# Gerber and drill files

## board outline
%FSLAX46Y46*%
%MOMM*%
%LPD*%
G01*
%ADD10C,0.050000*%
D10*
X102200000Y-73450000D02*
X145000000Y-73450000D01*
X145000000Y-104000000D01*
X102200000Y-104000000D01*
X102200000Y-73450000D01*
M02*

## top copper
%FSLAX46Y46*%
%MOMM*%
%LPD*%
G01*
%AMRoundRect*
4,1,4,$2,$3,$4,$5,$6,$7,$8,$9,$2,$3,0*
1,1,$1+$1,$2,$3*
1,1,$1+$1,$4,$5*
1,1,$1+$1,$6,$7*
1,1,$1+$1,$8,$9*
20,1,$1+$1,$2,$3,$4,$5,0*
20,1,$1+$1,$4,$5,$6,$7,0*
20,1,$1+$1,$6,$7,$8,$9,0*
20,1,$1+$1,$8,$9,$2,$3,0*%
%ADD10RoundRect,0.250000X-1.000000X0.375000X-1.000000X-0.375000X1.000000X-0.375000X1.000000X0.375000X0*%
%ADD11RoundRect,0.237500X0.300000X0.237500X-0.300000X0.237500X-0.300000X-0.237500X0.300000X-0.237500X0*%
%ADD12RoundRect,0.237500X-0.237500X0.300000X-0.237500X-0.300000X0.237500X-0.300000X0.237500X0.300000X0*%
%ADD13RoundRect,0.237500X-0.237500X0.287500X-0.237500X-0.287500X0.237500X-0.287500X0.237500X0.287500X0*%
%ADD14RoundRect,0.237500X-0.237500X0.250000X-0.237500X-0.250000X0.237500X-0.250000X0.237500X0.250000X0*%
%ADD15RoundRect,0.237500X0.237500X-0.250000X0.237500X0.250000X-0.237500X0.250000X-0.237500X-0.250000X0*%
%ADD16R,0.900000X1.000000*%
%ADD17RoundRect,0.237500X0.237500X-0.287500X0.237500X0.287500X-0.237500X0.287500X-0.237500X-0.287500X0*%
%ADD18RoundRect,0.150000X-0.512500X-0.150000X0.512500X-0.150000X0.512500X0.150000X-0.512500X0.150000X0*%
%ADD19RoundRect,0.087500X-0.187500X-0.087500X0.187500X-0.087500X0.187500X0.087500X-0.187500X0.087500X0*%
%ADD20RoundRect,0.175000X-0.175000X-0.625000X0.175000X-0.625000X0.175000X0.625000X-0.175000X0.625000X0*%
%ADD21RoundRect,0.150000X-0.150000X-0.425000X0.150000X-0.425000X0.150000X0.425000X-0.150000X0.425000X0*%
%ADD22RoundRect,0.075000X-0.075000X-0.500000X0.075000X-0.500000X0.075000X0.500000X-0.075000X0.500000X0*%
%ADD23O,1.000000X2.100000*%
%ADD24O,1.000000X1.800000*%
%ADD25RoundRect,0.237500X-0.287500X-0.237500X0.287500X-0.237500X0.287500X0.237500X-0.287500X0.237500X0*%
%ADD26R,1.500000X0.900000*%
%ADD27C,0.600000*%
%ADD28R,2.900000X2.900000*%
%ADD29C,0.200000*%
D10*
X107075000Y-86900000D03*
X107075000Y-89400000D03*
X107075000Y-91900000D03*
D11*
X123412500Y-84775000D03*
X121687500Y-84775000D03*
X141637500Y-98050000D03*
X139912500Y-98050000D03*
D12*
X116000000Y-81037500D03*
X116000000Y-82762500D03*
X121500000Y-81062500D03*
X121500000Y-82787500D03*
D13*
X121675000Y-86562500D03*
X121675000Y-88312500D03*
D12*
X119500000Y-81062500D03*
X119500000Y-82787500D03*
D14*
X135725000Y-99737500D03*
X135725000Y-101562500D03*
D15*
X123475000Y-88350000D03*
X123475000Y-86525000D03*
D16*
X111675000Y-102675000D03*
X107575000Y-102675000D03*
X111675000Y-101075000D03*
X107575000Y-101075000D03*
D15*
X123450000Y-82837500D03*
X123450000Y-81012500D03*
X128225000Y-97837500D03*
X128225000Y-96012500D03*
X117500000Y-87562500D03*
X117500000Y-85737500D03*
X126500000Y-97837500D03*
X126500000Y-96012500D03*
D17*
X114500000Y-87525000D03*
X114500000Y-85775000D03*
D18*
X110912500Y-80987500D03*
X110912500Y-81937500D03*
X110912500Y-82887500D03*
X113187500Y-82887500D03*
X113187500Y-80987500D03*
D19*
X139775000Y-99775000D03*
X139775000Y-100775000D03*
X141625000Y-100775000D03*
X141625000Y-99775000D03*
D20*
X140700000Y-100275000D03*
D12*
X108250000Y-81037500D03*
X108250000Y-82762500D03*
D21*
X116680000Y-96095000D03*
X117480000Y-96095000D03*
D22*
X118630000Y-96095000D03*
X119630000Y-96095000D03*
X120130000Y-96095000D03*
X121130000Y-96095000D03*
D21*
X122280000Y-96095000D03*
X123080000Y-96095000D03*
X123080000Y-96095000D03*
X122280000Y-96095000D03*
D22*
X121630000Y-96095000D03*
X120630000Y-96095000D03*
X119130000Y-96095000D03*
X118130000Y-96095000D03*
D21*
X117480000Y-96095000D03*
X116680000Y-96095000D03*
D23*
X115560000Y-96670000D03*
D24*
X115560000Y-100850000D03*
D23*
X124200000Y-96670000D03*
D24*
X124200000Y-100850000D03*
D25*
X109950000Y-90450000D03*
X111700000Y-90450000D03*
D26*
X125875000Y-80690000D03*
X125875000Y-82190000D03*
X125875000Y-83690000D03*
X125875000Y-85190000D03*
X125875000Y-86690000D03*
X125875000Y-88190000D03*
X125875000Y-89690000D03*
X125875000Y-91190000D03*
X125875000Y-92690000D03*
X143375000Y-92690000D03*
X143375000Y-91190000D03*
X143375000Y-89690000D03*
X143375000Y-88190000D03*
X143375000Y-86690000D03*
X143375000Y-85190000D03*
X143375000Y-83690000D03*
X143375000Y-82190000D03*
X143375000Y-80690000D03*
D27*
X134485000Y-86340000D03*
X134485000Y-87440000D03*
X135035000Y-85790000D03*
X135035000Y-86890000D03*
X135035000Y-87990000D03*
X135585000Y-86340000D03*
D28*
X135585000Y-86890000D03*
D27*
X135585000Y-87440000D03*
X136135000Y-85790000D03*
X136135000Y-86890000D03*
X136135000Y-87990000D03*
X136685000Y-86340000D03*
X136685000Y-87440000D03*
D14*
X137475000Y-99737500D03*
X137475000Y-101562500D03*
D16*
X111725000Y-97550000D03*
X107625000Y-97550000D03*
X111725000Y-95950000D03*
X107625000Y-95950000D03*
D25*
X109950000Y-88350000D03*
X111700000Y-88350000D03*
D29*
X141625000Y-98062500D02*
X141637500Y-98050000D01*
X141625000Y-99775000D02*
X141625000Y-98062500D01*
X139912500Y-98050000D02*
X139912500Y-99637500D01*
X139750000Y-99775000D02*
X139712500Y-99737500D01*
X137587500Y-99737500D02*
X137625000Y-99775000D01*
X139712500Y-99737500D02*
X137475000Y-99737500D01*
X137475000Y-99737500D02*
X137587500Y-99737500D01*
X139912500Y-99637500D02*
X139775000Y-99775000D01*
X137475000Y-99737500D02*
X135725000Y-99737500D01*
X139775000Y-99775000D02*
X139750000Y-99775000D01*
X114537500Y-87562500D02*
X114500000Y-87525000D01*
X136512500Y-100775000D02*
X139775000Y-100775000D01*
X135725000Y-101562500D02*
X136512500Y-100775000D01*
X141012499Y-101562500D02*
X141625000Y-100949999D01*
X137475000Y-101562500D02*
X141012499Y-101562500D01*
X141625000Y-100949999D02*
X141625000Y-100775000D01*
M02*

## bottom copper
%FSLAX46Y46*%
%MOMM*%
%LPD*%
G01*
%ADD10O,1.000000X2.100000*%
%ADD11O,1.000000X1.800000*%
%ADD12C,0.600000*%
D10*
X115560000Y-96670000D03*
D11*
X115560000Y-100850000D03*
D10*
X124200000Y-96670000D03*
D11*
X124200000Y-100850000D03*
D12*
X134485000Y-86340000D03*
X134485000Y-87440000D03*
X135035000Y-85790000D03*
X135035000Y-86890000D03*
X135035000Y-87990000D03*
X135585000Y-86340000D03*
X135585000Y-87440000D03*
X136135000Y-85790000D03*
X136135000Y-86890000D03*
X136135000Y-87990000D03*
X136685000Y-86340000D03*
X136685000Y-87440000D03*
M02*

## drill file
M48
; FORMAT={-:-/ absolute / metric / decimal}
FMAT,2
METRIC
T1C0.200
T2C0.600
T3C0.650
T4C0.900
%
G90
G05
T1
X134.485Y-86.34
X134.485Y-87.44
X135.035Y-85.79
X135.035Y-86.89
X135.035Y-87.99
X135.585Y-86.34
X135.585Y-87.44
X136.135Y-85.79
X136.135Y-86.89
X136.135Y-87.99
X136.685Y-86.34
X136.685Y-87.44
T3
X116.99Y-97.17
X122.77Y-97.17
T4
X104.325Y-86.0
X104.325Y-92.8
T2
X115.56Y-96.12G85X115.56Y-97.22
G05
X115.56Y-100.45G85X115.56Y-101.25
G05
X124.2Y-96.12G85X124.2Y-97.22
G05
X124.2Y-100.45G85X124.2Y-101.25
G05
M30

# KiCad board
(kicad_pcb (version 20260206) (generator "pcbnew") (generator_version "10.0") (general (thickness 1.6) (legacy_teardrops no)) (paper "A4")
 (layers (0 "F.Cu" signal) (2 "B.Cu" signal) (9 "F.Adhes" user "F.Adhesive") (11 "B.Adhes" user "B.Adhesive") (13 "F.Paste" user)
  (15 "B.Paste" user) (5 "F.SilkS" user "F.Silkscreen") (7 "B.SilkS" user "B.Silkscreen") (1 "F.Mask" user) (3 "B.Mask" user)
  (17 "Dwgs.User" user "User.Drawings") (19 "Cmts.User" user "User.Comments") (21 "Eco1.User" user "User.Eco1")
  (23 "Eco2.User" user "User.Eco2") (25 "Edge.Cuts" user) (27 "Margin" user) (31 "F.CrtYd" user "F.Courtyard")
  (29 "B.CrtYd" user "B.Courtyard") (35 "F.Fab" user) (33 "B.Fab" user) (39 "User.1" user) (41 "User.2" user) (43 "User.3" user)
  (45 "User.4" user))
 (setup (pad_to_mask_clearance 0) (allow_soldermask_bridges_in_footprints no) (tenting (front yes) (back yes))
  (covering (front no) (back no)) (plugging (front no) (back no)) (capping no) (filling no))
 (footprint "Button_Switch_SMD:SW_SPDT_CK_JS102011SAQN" (layer "F.Cu") (at 104.325 89.4 -90)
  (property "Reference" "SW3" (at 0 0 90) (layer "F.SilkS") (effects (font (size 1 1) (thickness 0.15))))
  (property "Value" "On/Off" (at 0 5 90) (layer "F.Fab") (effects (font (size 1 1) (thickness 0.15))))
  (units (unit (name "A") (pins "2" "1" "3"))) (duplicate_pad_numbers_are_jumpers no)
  (pad "" np_thru_hole circle (at -3.4 0 270) (size 0.9 0.9) (drill 0.9) (layers "*.Cu" "*.Mask"))
  (pad "" np_thru_hole circle (at 3.4 0 270) (size 0.9 0.9) (drill 0.9) (layers "*.Cu" "*.Mask"))
  (pad "1" smd roundrect (at -2.5 -2.75 270) (size 1.25 2.5) (layers "F.Cu" "F.Mask" "F.Paste") (roundrect_rratio 0.2) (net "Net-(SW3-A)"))
  (pad "2" smd roundrect (at 0 -2.75 270) (size 1.25 2.5) (layers "F.Cu" "F.Mask" "F.Paste") (roundrect_rratio 0.2) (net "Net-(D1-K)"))
  (pad "3" smd roundrect (at 2.5 -2.75 270) (size 1.25 2.5) (layers "F.Cu" "F.Mask" "F.Paste") (roundrect_rratio 0.2)
   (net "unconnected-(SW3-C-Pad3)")))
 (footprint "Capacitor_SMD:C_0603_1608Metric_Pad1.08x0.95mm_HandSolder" (layer "F.Cu") (at 122.55 84.775 180)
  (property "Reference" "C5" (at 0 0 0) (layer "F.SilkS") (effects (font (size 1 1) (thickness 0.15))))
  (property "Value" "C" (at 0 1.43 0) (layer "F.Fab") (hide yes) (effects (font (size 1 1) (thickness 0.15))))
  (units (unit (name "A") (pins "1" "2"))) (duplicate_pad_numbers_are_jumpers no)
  (pad "1" smd roundrect (at -0.8625 0 180) (size 1.075 0.95) (layers "F.Cu" "F.Mask" "F.Paste") (roundrect_rratio 0.25) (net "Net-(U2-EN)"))
  (pad "2" smd roundrect (at 0.8625 0 180) (size 1.075 0.95) (layers "F.Cu" "F.Mask" "F.Paste") (roundrect_rratio 0.25) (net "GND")))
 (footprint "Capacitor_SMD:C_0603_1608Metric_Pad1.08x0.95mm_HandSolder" (layer "F.Cu") (at 140.775 98.05 180)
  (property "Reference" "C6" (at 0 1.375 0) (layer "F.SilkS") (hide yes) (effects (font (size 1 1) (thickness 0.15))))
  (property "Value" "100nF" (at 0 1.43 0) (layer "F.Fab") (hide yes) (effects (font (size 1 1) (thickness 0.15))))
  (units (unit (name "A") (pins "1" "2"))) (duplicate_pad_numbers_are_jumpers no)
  (pad "1" smd roundrect (at -0.8625 0 180) (size 1.075 0.95) (layers "F.Cu" "F.Mask" "F.Paste") (roundrect_rratio 0.25) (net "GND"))
  (pad "2" smd roundrect (at 0.8625 0 180) (size 1.075 0.95) (layers "F.Cu" "F.Mask" "F.Paste") (roundrect_rratio 0.25) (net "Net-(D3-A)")))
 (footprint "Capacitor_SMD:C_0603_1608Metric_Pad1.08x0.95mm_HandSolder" (layer "F.Cu") (at 116 81.9 -90)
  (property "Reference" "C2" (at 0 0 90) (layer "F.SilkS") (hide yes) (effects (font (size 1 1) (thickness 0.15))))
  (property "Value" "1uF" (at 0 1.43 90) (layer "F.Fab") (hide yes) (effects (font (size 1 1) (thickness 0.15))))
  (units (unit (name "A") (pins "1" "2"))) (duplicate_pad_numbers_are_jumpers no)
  (pad "1" smd roundrect (at -0.8625 0 270) (size 1.075 0.95) (layers "F.Cu" "F.Mask" "F.Paste") (roundrect_rratio 0.25) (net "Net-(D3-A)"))
  (pad "2" smd roundrect (at 0.8625 0 270) (size 1.075 0.95) (layers "F.Cu" "F.Mask" "F.Paste") (roundrect_rratio 0.25) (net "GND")))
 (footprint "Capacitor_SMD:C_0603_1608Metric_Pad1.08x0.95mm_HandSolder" (layer "F.Cu") (at 121.5 81.925 -90)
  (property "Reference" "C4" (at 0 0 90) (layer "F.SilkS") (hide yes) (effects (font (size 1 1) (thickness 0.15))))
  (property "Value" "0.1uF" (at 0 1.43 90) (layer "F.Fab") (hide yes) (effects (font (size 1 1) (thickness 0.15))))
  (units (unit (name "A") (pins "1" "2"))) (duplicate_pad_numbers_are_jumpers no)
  (pad "1" smd roundrect (at -0.8625 0 270) (size 1.075 0.95) (layers "F.Cu" "F.Mask" "F.Paste") (roundrect_rratio 0.25) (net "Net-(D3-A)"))
  (pad "2" smd roundrect (at 0.8625 0 270) (size 1.075 0.95) (layers "F.Cu" "F.Mask" "F.Paste") (roundrect_rratio 0.25) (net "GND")))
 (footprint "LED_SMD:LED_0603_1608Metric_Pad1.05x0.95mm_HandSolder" (layer "F.Cu") (at 121.675 87.4375 -90)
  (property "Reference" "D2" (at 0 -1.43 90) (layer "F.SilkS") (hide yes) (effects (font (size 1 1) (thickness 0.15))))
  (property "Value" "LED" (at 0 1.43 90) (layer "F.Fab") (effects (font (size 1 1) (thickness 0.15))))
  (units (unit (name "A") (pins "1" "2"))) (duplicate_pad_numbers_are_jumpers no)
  (pad "1" smd roundrect (at -0.875 0 270) (size 1.05 0.95) (layers "F.Cu" "F.Mask" "F.Paste") (roundrect_rratio 0.25) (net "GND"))
  (pad "2" smd roundrect (at 0.875 0 270) (size 1.05 0.95) (layers "F.Cu" "F.Mask" "F.Paste") (roundrect_rratio 0.25) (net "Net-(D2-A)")))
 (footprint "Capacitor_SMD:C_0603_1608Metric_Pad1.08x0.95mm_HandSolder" (layer "F.Cu") (at 119.5 81.925 -90)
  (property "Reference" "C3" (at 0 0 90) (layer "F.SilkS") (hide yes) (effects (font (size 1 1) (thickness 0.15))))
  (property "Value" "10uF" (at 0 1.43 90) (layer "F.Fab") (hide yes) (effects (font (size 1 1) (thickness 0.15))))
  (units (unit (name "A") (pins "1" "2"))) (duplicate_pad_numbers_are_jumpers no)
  (pad "1" smd roundrect (at -0.8625 0 270) (size 1.075 0.95) (layers "F.Cu" "F.Mask" "F.Paste") (roundrect_rratio 0.25) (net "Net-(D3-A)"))
  (pad "2" smd roundrect (at 0.8625 0 270) (size 1.075 0.95) (layers "F.Cu" "F.Mask" "F.Paste") (roundrect_rratio 0.25) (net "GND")))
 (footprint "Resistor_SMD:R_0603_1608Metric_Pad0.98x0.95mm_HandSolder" (layer "F.Cu") (at 135.725 100.65 -90)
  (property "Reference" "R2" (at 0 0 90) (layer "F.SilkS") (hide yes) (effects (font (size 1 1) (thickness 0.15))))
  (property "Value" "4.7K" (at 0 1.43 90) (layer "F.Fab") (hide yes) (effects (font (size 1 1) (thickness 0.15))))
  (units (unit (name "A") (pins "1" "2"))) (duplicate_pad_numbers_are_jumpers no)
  (pad "1" smd roundrect (at -0.9125 0 270) (size 0.975 0.95) (layers "F.Cu" "F.Mask" "F.Paste") (roundrect_rratio 0.25) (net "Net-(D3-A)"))
  (pad "2" smd roundrect (at 0.9125 0 270) (size 0.975 0.95) (layers "F.Cu" "F.Mask" "F.Paste") (roundrect_rratio 0.25) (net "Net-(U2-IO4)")))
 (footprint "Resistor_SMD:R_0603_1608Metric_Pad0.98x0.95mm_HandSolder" (layer "F.Cu") (at 123.475 87.4375 90)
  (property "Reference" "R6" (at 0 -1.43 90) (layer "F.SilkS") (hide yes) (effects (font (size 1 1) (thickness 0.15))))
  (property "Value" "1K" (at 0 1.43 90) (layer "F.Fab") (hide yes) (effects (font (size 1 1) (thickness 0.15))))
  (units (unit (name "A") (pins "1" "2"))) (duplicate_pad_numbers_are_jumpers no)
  (pad "1" smd roundrect (at -0.9125 0 90) (size 0.975 0.95) (layers "F.Cu" "F.Mask" "F.Paste") (roundrect_rratio 0.25) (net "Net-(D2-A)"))
  (pad "2" smd roundrect (at 0.9125 0 90) (size 0.975 0.95) (layers "F.Cu" "F.Mask" "F.Paste") (roundrect_rratio 0.25) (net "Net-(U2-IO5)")))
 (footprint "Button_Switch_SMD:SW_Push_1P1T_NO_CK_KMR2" (layer "F.Cu") (at 109.625 101.875 180)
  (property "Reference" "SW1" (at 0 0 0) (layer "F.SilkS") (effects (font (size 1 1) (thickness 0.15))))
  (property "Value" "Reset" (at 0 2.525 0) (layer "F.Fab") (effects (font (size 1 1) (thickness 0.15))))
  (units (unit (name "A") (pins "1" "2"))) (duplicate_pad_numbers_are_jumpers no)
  (pad "1" smd rect (at -2.05 -0.8 180) (size 0.9 1) (layers "F.Cu" "F.Mask" "F.Paste") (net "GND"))
  (pad "1" smd rect (at 2.05 -0.8 180) (size 0.9 1) (layers "F.Cu" "F.Mask" "F.Paste") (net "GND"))
  (pad "2" smd rect (at -2.05 0.8 180) (size 0.9 1) (layers "F.Cu" "F.Mask" "F.Paste") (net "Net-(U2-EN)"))
  (pad "2" smd rect (at 2.05 0.8 180) (size 0.9 1) (layers "F.Cu" "F.Mask" "F.Paste") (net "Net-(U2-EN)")))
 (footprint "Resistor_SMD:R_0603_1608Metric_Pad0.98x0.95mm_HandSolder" (layer "F.Cu") (at 123.45 81.925 90)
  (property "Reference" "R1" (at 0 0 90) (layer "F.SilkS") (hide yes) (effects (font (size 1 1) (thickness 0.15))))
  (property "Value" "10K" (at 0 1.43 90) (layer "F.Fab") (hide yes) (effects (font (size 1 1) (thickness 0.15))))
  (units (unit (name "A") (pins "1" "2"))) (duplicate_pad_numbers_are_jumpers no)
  (pad "1" smd roundrect (at -0.9125 0 90) (size 0.975 0.95) (layers "F.Cu" "F.Mask" "F.Paste") (roundrect_rratio 0.25) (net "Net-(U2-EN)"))
  (pad "2" smd roundrect (at 0.9125 0 90) (size 0.975 0.95) (layers "F.Cu" "F.Mask" "F.Paste") (roundrect_rratio 0.25) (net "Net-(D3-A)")))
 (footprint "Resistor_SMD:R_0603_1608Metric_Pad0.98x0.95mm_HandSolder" (layer "F.Cu") (at 128.225 96.925 90)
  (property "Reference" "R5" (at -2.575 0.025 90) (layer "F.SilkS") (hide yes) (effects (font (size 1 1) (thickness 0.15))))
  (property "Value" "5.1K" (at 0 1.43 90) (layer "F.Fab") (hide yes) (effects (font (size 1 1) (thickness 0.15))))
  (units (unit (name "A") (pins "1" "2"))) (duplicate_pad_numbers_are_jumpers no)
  (pad "1" smd roundrect (at -0.9125 0 90) (size 0.975 0.95) (layers "F.Cu" "F.Mask" "F.Paste") (roundrect_rratio 0.25) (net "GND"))
  (pad "2" smd roundrect (at 0.9125 0 90) (size 0.975 0.95) (layers "F.Cu" "F.Mask" "F.Paste") (roundrect_rratio 0.25) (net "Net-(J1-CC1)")))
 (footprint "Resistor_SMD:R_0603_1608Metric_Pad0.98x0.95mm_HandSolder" (layer "F.Cu") (at 117.5 86.65 90)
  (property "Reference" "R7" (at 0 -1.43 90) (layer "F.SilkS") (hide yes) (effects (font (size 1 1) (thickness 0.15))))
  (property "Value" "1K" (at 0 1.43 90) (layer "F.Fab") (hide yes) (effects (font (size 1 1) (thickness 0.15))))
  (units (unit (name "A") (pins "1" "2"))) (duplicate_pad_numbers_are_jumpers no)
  (pad "1" smd roundrect (at -0.9125 0 90) (size 0.975 0.95) (layers "F.Cu" "F.Mask" "F.Paste") (roundrect_rratio 0.25) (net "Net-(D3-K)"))
  (pad "2" smd roundrect (at 0.9125 0 90) (size 0.975 0.95) (layers "F.Cu" "F.Mask" "F.Paste") (roundrect_rratio 0.25) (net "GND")))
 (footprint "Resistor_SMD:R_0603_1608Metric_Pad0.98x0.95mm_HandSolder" (layer "F.Cu") (at 126.5 96.925 90)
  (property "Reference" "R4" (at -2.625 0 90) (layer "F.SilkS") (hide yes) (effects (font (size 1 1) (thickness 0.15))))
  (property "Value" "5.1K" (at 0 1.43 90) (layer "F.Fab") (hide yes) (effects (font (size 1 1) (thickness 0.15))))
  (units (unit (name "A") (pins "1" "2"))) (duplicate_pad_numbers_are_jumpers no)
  (pad "1" smd roundrect (at -0.9125 0 90) (size 0.975 0.95) (layers "F.Cu" "F.Mask" "F.Paste") (roundrect_rratio 0.25) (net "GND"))
  (pad "2" smd roundrect (at 0.9125 0 90) (size 0.975 0.95) (layers "F.Cu" "F.Mask" "F.Paste") (roundrect_rratio 0.25) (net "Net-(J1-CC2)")))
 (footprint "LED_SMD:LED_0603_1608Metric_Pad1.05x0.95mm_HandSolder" (layer "F.Cu") (at 114.5 86.65 90)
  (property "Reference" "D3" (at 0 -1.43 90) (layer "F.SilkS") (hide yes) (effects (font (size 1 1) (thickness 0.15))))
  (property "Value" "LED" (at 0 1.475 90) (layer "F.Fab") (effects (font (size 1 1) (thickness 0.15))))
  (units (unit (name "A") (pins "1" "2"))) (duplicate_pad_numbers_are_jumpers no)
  (pad "1" smd roundrect (at -0.875 0 90) (size 1.05 0.95) (layers "F.Cu" "F.Mask" "F.Paste") (roundrect_rratio 0.25) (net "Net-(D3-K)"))
  (pad "2" smd roundrect (at 0.875 0 90) (size 1.05 0.95) (layers "F.Cu" "F.Mask" "F.Paste") (roundrect_rratio 0.25) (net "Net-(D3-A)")))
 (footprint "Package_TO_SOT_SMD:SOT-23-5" (layer "F.Cu") (at 112.05 81.9375)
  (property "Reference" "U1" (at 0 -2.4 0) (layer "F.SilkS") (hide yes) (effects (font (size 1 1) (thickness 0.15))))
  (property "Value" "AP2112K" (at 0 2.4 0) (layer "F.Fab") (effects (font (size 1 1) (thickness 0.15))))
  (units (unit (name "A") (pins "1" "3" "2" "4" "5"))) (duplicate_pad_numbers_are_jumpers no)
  (pad "1" smd roundrect (at -1.1375 -0.95) (size 1.325 0.6) (layers "F.Cu" "F.Mask" "F.Paste") (roundrect_rratio 0.25) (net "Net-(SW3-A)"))
  (pad "2" smd roundrect (at -1.1375 0) (size 1.325 0.6) (layers "F.Cu" "F.Mask" "F.Paste") (roundrect_rratio 0.25) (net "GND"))
  (pad "3" smd roundrect (at -1.1375 0.95) (size 1.325 0.6) (layers "F.Cu" "F.Mask" "F.Paste") (roundrect_rratio 0.25) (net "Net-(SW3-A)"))
  (pad "4" smd roundrect (at 1.1375 0.95) (size 1.325 0.6) (layers "F.Cu" "F.Mask" "F.Paste") (roundrect_rratio 0.25)
   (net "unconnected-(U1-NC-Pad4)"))
  (pad "5" smd roundrect (at 1.1375 -0.95) (size 1.325 0.6) (layers "F.Cu" "F.Mask" "F.Paste") (roundrect_rratio 0.25) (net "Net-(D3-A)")))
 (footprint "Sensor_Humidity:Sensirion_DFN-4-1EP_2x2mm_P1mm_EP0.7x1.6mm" (layer "F.Cu") (at 140.7 100.275)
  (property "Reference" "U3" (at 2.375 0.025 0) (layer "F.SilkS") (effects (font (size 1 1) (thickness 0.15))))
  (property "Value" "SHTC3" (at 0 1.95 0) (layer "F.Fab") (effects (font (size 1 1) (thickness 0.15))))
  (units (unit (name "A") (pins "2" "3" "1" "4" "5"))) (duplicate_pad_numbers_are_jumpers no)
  (pad "" smd roundrect (at -1.025 -0.5) (size 0.55 0.35) (layers "F.Paste") (roundrect_rratio 0.25))
  (pad "" smd roundrect (at -1.025 0.5) (size 0.55 0.35) (layers "F.Paste") (roundrect_rratio 0.25))
  (pad "" smd roundrect (at 0 0) (size 0.5 1.4) (layers "F.Paste") (roundrect_rratio 0.25))
  (pad "" smd roundrect (at 1.025 -0.5 180) (size 0.55 0.35) (layers "F.Paste") (roundrect_rratio 0.25))
  (pad "" smd roundrect (at 1.025 0.5 180) (size 0.55 0.35) (layers "F.Paste") (roundrect_rratio 0.25))
  (pad "1" smd roundrect (at -0.925 -0.5) (size 0.55 0.35) (layers "F.Cu" "F.Mask") (roundrect_rratio 0.25) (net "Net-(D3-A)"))
  (pad "2" smd roundrect (at -0.925 0.5) (size 0.55 0.35) (layers "F.Cu" "F.Mask") (roundrect_rratio 0.25) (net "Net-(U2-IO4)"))
  (pad "3" smd roundrect (at 0.925 0.5) (size 0.55 0.35) (layers "F.Cu" "F.Mask") (roundrect_rratio 0.25) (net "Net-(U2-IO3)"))
  (pad "4" smd roundrect (at 0.925 -0.5) (size 0.55 0.35) (layers "F.Cu" "F.Mask") (roundrect_rratio 0.25) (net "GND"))
  (pad "5" smd roundrect (at 0 0) (size 0.7 1.6) (layers "F.Cu" "F.Mask") (roundrect_rratio 0.25) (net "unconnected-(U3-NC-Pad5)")))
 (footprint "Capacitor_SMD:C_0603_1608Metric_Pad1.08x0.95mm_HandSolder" (layer "F.Cu") (at 108.25 81.9 -90)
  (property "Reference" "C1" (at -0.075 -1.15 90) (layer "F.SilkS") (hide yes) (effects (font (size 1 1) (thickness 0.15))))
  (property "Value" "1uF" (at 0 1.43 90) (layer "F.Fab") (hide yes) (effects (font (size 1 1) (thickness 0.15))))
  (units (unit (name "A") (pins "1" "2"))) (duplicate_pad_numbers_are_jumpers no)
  (pad "1" smd roundrect (at -0.8625 0 270) (size 1.075 0.95) (layers "F.Cu" "F.Mask" "F.Paste") (roundrect_rratio 0.25) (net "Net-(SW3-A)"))
  (pad "2" smd roundrect (at 0.8625 0 270) (size 1.075 0.95) (layers "F.Cu" "F.Mask" "F.Paste") (roundrect_rratio 0.25) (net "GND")))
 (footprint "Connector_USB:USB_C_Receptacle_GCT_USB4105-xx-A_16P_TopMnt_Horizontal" (layer "F.Cu") (at 119.88 99.775)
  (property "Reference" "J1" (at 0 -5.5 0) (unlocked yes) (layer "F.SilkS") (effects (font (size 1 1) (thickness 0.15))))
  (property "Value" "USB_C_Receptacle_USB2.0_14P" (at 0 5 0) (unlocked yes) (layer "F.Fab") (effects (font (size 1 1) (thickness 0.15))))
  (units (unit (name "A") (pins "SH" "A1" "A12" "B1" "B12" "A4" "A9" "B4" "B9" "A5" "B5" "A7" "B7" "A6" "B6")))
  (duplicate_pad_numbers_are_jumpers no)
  (pad "" np_thru_hole circle (at -2.89 -2.605) (size 0.65 0.65) (drill 0.65) (layers "*.Cu" "*.Mask"))
  (pad "" np_thru_hole circle (at 2.89 -2.605) (size 0.65 0.65) (drill 0.65) (layers "*.Cu" "*.Mask"))
  (pad "A1" smd roundrect (at -3.2 -3.68) (size 0.6 1.15) (layers "F.Cu" "F.Mask" "F.Paste") (roundrect_rratio 0.25) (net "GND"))
  (pad "A4" smd roundrect (at -2.4 -3.68) (size 0.6 1.15) (layers "F.Cu" "F.Mask" "F.Paste") (roundrect_rratio 0.25) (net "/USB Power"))
  (pad "A5" smd roundrect (at -1.25 -3.68) (size 0.3 1.15) (layers "F.Cu" "F.Mask" "F.Paste") (roundrect_rratio 0.25) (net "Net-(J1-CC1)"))
  (pad "A6" smd roundrect (at -0.25 -3.68) (size 0.3 1.15) (layers "F.Cu" "F.Mask" "F.Paste") (roundrect_rratio 0.25) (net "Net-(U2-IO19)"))
  (pad "A7" smd roundrect (at 0.25 -3.68) (size 0.3 1.15) (layers "F.Cu" "F.Mask" "F.Paste") (roundrect_rratio 0.25) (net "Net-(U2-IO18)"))
  (pad "A8" smd roundrect (at 1.25 -3.68) (size 0.3 1.15) (layers "F.Cu" "F.Mask" "F.Paste") (roundrect_rratio 0.25))
  (pad "A9" smd roundrect (at 2.4 -3.68) (size 0.6 1.15) (layers "F.Cu" "F.Mask" "F.Paste") (roundrect_rratio 0.25) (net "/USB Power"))
  (pad "A12" smd roundrect (at 3.2 -3.68) (size 0.6 1.15) (layers "F.Cu" "F.Mask" "F.Paste") (roundrect_rratio 0.25) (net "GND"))
  (pad "B1" smd roundrect (at 3.2 -3.68) (size 0.6 1.15) (layers "F.Cu" "F.Mask" "F.Paste") (roundrect_rratio 0.25) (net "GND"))
  (pad "B4" smd roundrect (at 2.4 -3.68) (size 0.6 1.15) (layers "F.Cu" "F.Mask" "F.Paste") (roundrect_rratio 0.25) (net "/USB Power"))
  (pad "B5" smd roundrect (at 1.75 -3.68) (size 0.3 1.15) (layers "F.Cu" "F.Mask" "F.Paste") (roundrect_rratio 0.25) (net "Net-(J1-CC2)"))
  (pad "B6" smd roundrect (at 0.75 -3.68) (size 0.3 1.15) (layers "F.Cu" "F.Mask" "F.Paste") (roundrect_rratio 0.25) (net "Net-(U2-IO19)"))
  (pad "B7" smd roundrect (at -0.75 -3.68) (size 0.3 1.15) (layers "F.Cu" "F.Mask" "F.Paste") (roundrect_rratio 0.25) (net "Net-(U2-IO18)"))
  (pad "B8" smd roundrect (at -1.75 -3.68) (size 0.3 1.15) (layers "F.Cu" "F.Mask" "F.Paste") (roundrect_rratio 0.25))
  (pad "B9" smd roundrect (at -2.4 -3.68) (size 0.6 1.15) (layers "F.Cu" "F.Mask" "F.Paste") (roundrect_rratio 0.25) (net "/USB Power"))
  (pad "B12" smd roundrect (at -3.2 -3.68) (size 0.6 1.15) (layers "F.Cu" "F.Mask" "F.Paste") (roundrect_rratio 0.25) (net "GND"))
  (pad "SH" thru_hole oval (at -4.32 -3.105) (size 1 2.1) (drill oval 0.6 1.7) (layers "*.Cu" "*.Mask" "F.Paste") (remove_unused_layers no)
   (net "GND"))
  (pad "SH" thru_hole oval (at -4.32 1.075) (size 1 1.8) (drill oval 0.6 1.4) (layers "*.Cu" "*.Mask" "F.Paste") (remove_unused_layers no)
   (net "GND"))
  (pad "SH" thru_hole oval (at 4.32 -3.105) (size 1 2.1) (drill oval 0.6 1.7) (layers "*.Cu" "*.Mask" "F.Paste") (remove_unused_layers no)
   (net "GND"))
  (pad "SH" thru_hole oval (at 4.32 1.075) (size 1 1.8) (drill oval 0.6 1.4) (layers "*.Cu" "*.Mask" "F.Paste") (remove_unused_layers no)
   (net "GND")))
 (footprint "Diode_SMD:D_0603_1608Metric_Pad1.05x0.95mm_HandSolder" (layer "F.Cu") (at 110.825 90.45)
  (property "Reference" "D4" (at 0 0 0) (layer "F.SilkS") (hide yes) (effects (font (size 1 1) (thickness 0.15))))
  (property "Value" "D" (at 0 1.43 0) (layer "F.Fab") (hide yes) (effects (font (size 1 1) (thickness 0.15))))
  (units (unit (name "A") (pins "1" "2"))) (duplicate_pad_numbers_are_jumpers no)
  (pad "1" smd roundrect (at -0.875 0) (size 1.05 0.95) (layers "F.Cu" "F.Mask" "F.Paste") (roundrect_rratio 0.25) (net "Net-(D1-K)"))
  (pad "2" smd roundrect (at 0.875 0) (size 1.05 0.95) (layers "F.Cu" "F.Mask" "F.Paste") (roundrect_rratio 0.25) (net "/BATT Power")))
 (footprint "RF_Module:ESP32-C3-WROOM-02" (layer "F.Cu") (at 134.625 86.69)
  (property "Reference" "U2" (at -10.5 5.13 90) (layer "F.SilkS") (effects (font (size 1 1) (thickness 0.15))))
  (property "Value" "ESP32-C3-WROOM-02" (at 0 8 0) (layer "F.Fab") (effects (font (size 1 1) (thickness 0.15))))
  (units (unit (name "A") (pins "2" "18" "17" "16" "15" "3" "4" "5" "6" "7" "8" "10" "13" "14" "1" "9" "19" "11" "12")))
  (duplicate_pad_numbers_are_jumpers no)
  (pad "" smd rect (at -0.14 -0.9) (size 0.7 0.7) (layers "F.Paste"))
  (pad "" smd rect (at -0.14 0.2) (size 0.7 0.7) (layers "F.Paste"))
  (pad "" smd rect (at -0.14 1.3) (size 0.7 0.7) (layers "F.Paste"))
  (pad "" smd rect (at 0.96 -0.9) (size 0.7 0.7) (layers "F.Paste"))
  (pad "" smd rect (at 0.96 0.2) (size 0.7 0.7) (layers "F.Paste"))
  (pad "" smd rect (at 0.96 1.3) (size 0.7 0.7) (layers "F.Paste"))
  (pad "" smd rect (at 2.06 -0.9) (size 0.7 0.7) (layers "F.Paste"))
  (pad "" smd rect (at 2.06 0.2) (size 0.7 0.7) (layers "F.Paste"))
  (pad "" smd rect (at 2.06 1.3) (size 0.7 0.7) (layers "F.Paste"))
  (pad "1" smd rect (at -8.75 -6) (size 1.5 0.9) (layers "F.Cu" "F.Mask" "F.Paste") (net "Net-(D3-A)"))
  (pad "2" smd rect (at -8.75 -4.5) (size 1.5 0.9) (layers "F.Cu" "F.Mask" "F.Paste") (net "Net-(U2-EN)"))
  (pad "3" smd rect (at -8.75 -3) (size 1.5 0.9) (layers "F.Cu" "F.Mask" "F.Paste") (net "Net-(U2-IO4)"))
  (pad "4" smd rect (at -8.75 -1.5) (size 1.5 0.9) (layers "F.Cu" "F.Mask" "F.Paste") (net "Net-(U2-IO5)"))
  (pad "5" smd rect (at -8.75 0) (size 1.5 0.9) (layers "F.Cu" "F.Mask" "F.Paste") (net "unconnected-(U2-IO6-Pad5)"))
  (pad "6" smd rect (at -8.75 1.5) (size 1.5 0.9) (layers "F.Cu" "F.Mask" "F.Paste") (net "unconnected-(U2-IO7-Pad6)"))
  (pad "7" smd rect (at -8.75 3) (size 1.5 0.9) (layers "F.Cu" "F.Mask" "F.Paste") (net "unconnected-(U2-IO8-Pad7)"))
  (pad "8" smd rect (at -8.75 4.5) (size 1.5 0.9) (layers "F.Cu" "F.Mask" "F.Paste") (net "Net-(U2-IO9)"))
  (pad "9" smd rect (at -8.75 6) (size 1.5 0.9) (layers "F.Cu" "F.Mask" "F.Paste") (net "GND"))
  (pad "10" smd rect (at 8.75 6) (size 1.5 0.9) (layers "F.Cu" "F.Mask" "F.Paste") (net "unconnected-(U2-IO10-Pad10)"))
  (pad "11" smd rect (at 8.75 4.5) (size 1.5 0.9) (layers "F.Cu" "F.Mask" "F.Paste") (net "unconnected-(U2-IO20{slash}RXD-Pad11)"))
  (pad "12" smd rect (at 8.75 3) (size 1.5 0.9) (layers "F.Cu" "F.Mask" "F.Paste") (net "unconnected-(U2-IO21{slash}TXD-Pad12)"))
  (pad "13" smd rect (at 8.75 1.5) (size 1.5 0.9) (layers "F.Cu" "F.Mask" "F.Paste") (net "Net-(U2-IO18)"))
  (pad "14" smd rect (at 8.75 0) (size 1.5 0.9) (layers "F.Cu" "F.Mask" "F.Paste") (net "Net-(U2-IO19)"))
  (pad "15" smd rect (at 8.75 -1.5) (size 1.5 0.9) (layers "F.Cu" "F.Mask" "F.Paste") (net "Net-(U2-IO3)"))
  (pad "16" smd rect (at 8.75 -3) (size 1.5 0.9) (layers "F.Cu" "F.Mask" "F.Paste") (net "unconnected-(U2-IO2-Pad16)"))
  (pad "17" smd rect (at 8.75 -4.5) (size 1.5 0.9) (layers "F.Cu" "F.Mask" "F.Paste") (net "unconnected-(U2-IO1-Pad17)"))
  (pad "18" smd rect (at 8.75 -6) (size 1.5 0.9) (layers "F.Cu" "F.Mask" "F.Paste") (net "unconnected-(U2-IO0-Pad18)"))
  (pad "19" thru_hole circle (at -0.14 -0.35) (size 0.6 0.6) (drill 0.2) (layers "*.Cu" "F.Mask") (remove_unused_layers no) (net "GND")
   (zone_connect 2))
  (pad "19" thru_hole circle (at -0.14 0.75) (size 0.6 0.6) (drill 0.2) (layers "*.Cu" "F.Mask") (remove_unused_layers no) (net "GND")
   (zone_connect 2))
  (pad "19" thru_hole circle (at 0.41 -0.9) (size 0.6 0.6) (drill 0.2) (layers "*.Cu" "F.Mask") (remove_unused_layers no) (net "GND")
   (zone_connect 2))
  (pad "19" thru_hole circle (at 0.41 0.2) (size 0.6 0.6) (drill 0.2) (layers "*.Cu" "F.Mask") (remove_unused_layers no) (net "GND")
   (zone_connect 2))
  (pad "19" thru_hole circle (at 0.41 1.3) (size 0.6 0.6) (drill 0.2) (layers "*.Cu" "F.Mask") (remove_unused_layers no) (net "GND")
   (zone_connect 2))
  (pad "19" thru_hole circle (at 0.96 -0.35) (size 0.6 0.6) (drill 0.2) (layers "*.Cu" "F.Mask") (remove_unused_layers no) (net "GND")
   (zone_connect 2))
  (pad "19" smd rect (at 0.96 0.2) (size 2.9 2.9) (layers "F.Cu" "F.Mask") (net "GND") (zone_connect 2))
  (pad "19" thru_hole circle (at 0.96 0.75) (size 0.6 0.6) (drill 0.2) (layers "*.Cu" "F.Mask") (remove_unused_layers no) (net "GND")
   (zone_connect 2))
  (pad "19" thru_hole circle (at 1.51 -0.9) (size 0.6 0.6) (drill 0.2) (layers "*.Cu" "F.Mask") (remove_unused_layers no) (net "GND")
   (zone_connect 2))
  (pad "19" thru_hole circle (at 1.51 0.2) (size 0.6 0.6) (drill 0.2) (layers "*.Cu" "F.Mask") (remove_unused_layers no) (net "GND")
   (zone_connect 2))
  (pad "19" thru_hole circle (at 1.51 1.3) (size 0.6 0.6) (drill 0.2) (layers "*.Cu" "F.Mask") (remove_unused_layers no) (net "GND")
   (zone_connect 2))
  (pad "19" thru_hole circle (at 2.06 -0.35) (size 0.6 0.6) (drill 0.2) (layers "*.Cu" "F.Mask") (remove_unused_layers no) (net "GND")
   (zone_connect 2))
  (pad "19" thru_hole circle (at 2.06 0.75) (size 0.6 0.6) (drill 0.2) (layers "*.Cu" "F.Mask") (remove_unused_layers no) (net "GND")
   (zone_connect 2))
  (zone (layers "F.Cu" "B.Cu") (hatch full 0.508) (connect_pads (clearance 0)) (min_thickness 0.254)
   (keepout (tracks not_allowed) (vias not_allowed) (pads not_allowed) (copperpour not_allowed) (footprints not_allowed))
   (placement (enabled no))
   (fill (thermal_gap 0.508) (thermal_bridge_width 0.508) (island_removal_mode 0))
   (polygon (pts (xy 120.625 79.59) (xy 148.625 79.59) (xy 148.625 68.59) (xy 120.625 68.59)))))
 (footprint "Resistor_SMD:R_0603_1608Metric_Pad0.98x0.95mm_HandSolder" (layer "F.Cu") (at 137.475 100.65 -90)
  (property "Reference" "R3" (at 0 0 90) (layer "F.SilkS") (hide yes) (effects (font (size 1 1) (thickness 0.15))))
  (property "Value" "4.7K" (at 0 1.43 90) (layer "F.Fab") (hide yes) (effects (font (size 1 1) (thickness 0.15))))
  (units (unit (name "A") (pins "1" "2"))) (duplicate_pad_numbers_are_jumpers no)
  (pad "1" smd roundrect (at -0.9125 0 270) (size 0.975 0.95) (layers "F.Cu" "F.Mask" "F.Paste") (roundrect_rratio 0.25) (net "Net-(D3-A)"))
  (pad "2" smd roundrect (at 0.9125 0 270) (size 0.975 0.95) (layers "F.Cu" "F.Mask" "F.Paste") (roundrect_rratio 0.25) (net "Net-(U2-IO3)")))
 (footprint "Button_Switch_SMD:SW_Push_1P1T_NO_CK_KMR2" (layer "F.Cu") (at 109.675 96.75 180)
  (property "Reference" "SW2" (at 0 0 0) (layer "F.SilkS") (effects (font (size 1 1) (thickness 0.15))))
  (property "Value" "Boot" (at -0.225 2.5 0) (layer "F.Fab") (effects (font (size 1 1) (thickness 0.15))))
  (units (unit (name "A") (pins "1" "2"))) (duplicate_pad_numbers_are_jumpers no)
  (pad "1" smd rect (at -2.05 -0.8 180) (size 0.9 1) (layers "F.Cu" "F.Mask" "F.Paste") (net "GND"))
  (pad "1" smd rect (at 2.05 -0.8 180) (size 0.9 1) (layers "F.Cu" "F.Mask" "F.Paste") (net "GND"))
  (pad "2" smd rect (at -2.05 0.8 180) (size 0.9 1) (layers "F.Cu" "F.Mask" "F.Paste") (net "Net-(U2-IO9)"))
  (pad "2" smd rect (at 2.05 0.8 180) (size 0.9 1) (layers "F.Cu" "F.Mask" "F.Paste") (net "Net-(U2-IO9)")))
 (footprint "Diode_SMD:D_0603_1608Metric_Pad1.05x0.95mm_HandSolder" (layer "F.Cu") (at 110.825 88.35)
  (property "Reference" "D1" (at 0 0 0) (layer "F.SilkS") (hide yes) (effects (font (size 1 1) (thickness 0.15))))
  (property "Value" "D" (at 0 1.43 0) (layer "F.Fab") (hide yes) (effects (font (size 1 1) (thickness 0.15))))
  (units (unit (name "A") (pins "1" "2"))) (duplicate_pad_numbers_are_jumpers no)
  (pad "1" smd roundrect (at -0.875 0) (size 1.05 0.95) (layers "F.Cu" "F.Mask" "F.Paste") (roundrect_rratio 0.25) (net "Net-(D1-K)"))
  (pad "2" smd roundrect (at 0.875 0) (size 1.05 0.95) (layers "F.Cu" "F.Mask" "F.Paste") (roundrect_rratio 0.25) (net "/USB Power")))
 (gr_rect (start 102.2 73.45) (end 145 104) (stroke (width 0.05) (type default)) (fill no) (layer "Edge.Cuts"))
 (segment (start 141.625 98.0625) (end 141.6375 98.05) (width 0.2) (layer "F.Cu") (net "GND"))
 (segment (start 141.625 99.775) (end 141.625 98.0625) (width 0.2) (layer "F.Cu") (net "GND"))
 (segment (start 139.9125 98.05) (end 139.9125 99.6375) (width 0.2) (layer "F.Cu") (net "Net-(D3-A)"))
 (segment (start 139.75 99.775) (end 139.7125 99.7375) (width 0.2) (layer "F.Cu") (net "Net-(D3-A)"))
 (segment (start 137.5875 99.7375) (end 137.625 99.775) (width 0.2) (layer "F.Cu") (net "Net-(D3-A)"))
 (segment (start 139.7125 99.7375) (end 137.475 99.7375) (width 0.2) (layer "F.Cu") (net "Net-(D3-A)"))
 (segment (start 137.475 99.7375) (end 137.5875 99.7375) (width 0.2) (layer "F.Cu") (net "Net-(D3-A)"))
 (segment (start 139.9125 99.6375) (end 139.775 99.775) (width 0.2) (layer "F.Cu") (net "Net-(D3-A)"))
 (segment (start 137.475 99.7375) (end 135.725 99.7375) (width 0.2) (layer "F.Cu") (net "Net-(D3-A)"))
 (segment (start 139.775 99.775) (end 139.75 99.775) (width 0.2) (layer "F.Cu") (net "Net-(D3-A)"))
 (segment (start 114.5375 87.5625) (end 114.5 87.525) (width 0.2) (layer "F.Cu") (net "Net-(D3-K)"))
 (segment (start 136.5125 100.775) (end 139.775 100.775) (width 0.2) (layer "F.Cu") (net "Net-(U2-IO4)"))
 (segment (start 135.725 101.5625) (end 136.5125 100.775) (width 0.2) (layer "F.Cu") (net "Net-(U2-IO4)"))
 (segment (start 141.012499 101.5625) (end 141.625 100.949999) (width 0.2) (layer "F.Cu") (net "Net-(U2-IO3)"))
 (segment (start 137.475 101.5625) (end 141.012499 101.5625) (width 0.2) (layer "F.Cu") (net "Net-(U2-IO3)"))
 (segment (start 141.625 100.949999) (end 141.625 100.775) (width 0.2) (layer "F.Cu") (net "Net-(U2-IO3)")))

